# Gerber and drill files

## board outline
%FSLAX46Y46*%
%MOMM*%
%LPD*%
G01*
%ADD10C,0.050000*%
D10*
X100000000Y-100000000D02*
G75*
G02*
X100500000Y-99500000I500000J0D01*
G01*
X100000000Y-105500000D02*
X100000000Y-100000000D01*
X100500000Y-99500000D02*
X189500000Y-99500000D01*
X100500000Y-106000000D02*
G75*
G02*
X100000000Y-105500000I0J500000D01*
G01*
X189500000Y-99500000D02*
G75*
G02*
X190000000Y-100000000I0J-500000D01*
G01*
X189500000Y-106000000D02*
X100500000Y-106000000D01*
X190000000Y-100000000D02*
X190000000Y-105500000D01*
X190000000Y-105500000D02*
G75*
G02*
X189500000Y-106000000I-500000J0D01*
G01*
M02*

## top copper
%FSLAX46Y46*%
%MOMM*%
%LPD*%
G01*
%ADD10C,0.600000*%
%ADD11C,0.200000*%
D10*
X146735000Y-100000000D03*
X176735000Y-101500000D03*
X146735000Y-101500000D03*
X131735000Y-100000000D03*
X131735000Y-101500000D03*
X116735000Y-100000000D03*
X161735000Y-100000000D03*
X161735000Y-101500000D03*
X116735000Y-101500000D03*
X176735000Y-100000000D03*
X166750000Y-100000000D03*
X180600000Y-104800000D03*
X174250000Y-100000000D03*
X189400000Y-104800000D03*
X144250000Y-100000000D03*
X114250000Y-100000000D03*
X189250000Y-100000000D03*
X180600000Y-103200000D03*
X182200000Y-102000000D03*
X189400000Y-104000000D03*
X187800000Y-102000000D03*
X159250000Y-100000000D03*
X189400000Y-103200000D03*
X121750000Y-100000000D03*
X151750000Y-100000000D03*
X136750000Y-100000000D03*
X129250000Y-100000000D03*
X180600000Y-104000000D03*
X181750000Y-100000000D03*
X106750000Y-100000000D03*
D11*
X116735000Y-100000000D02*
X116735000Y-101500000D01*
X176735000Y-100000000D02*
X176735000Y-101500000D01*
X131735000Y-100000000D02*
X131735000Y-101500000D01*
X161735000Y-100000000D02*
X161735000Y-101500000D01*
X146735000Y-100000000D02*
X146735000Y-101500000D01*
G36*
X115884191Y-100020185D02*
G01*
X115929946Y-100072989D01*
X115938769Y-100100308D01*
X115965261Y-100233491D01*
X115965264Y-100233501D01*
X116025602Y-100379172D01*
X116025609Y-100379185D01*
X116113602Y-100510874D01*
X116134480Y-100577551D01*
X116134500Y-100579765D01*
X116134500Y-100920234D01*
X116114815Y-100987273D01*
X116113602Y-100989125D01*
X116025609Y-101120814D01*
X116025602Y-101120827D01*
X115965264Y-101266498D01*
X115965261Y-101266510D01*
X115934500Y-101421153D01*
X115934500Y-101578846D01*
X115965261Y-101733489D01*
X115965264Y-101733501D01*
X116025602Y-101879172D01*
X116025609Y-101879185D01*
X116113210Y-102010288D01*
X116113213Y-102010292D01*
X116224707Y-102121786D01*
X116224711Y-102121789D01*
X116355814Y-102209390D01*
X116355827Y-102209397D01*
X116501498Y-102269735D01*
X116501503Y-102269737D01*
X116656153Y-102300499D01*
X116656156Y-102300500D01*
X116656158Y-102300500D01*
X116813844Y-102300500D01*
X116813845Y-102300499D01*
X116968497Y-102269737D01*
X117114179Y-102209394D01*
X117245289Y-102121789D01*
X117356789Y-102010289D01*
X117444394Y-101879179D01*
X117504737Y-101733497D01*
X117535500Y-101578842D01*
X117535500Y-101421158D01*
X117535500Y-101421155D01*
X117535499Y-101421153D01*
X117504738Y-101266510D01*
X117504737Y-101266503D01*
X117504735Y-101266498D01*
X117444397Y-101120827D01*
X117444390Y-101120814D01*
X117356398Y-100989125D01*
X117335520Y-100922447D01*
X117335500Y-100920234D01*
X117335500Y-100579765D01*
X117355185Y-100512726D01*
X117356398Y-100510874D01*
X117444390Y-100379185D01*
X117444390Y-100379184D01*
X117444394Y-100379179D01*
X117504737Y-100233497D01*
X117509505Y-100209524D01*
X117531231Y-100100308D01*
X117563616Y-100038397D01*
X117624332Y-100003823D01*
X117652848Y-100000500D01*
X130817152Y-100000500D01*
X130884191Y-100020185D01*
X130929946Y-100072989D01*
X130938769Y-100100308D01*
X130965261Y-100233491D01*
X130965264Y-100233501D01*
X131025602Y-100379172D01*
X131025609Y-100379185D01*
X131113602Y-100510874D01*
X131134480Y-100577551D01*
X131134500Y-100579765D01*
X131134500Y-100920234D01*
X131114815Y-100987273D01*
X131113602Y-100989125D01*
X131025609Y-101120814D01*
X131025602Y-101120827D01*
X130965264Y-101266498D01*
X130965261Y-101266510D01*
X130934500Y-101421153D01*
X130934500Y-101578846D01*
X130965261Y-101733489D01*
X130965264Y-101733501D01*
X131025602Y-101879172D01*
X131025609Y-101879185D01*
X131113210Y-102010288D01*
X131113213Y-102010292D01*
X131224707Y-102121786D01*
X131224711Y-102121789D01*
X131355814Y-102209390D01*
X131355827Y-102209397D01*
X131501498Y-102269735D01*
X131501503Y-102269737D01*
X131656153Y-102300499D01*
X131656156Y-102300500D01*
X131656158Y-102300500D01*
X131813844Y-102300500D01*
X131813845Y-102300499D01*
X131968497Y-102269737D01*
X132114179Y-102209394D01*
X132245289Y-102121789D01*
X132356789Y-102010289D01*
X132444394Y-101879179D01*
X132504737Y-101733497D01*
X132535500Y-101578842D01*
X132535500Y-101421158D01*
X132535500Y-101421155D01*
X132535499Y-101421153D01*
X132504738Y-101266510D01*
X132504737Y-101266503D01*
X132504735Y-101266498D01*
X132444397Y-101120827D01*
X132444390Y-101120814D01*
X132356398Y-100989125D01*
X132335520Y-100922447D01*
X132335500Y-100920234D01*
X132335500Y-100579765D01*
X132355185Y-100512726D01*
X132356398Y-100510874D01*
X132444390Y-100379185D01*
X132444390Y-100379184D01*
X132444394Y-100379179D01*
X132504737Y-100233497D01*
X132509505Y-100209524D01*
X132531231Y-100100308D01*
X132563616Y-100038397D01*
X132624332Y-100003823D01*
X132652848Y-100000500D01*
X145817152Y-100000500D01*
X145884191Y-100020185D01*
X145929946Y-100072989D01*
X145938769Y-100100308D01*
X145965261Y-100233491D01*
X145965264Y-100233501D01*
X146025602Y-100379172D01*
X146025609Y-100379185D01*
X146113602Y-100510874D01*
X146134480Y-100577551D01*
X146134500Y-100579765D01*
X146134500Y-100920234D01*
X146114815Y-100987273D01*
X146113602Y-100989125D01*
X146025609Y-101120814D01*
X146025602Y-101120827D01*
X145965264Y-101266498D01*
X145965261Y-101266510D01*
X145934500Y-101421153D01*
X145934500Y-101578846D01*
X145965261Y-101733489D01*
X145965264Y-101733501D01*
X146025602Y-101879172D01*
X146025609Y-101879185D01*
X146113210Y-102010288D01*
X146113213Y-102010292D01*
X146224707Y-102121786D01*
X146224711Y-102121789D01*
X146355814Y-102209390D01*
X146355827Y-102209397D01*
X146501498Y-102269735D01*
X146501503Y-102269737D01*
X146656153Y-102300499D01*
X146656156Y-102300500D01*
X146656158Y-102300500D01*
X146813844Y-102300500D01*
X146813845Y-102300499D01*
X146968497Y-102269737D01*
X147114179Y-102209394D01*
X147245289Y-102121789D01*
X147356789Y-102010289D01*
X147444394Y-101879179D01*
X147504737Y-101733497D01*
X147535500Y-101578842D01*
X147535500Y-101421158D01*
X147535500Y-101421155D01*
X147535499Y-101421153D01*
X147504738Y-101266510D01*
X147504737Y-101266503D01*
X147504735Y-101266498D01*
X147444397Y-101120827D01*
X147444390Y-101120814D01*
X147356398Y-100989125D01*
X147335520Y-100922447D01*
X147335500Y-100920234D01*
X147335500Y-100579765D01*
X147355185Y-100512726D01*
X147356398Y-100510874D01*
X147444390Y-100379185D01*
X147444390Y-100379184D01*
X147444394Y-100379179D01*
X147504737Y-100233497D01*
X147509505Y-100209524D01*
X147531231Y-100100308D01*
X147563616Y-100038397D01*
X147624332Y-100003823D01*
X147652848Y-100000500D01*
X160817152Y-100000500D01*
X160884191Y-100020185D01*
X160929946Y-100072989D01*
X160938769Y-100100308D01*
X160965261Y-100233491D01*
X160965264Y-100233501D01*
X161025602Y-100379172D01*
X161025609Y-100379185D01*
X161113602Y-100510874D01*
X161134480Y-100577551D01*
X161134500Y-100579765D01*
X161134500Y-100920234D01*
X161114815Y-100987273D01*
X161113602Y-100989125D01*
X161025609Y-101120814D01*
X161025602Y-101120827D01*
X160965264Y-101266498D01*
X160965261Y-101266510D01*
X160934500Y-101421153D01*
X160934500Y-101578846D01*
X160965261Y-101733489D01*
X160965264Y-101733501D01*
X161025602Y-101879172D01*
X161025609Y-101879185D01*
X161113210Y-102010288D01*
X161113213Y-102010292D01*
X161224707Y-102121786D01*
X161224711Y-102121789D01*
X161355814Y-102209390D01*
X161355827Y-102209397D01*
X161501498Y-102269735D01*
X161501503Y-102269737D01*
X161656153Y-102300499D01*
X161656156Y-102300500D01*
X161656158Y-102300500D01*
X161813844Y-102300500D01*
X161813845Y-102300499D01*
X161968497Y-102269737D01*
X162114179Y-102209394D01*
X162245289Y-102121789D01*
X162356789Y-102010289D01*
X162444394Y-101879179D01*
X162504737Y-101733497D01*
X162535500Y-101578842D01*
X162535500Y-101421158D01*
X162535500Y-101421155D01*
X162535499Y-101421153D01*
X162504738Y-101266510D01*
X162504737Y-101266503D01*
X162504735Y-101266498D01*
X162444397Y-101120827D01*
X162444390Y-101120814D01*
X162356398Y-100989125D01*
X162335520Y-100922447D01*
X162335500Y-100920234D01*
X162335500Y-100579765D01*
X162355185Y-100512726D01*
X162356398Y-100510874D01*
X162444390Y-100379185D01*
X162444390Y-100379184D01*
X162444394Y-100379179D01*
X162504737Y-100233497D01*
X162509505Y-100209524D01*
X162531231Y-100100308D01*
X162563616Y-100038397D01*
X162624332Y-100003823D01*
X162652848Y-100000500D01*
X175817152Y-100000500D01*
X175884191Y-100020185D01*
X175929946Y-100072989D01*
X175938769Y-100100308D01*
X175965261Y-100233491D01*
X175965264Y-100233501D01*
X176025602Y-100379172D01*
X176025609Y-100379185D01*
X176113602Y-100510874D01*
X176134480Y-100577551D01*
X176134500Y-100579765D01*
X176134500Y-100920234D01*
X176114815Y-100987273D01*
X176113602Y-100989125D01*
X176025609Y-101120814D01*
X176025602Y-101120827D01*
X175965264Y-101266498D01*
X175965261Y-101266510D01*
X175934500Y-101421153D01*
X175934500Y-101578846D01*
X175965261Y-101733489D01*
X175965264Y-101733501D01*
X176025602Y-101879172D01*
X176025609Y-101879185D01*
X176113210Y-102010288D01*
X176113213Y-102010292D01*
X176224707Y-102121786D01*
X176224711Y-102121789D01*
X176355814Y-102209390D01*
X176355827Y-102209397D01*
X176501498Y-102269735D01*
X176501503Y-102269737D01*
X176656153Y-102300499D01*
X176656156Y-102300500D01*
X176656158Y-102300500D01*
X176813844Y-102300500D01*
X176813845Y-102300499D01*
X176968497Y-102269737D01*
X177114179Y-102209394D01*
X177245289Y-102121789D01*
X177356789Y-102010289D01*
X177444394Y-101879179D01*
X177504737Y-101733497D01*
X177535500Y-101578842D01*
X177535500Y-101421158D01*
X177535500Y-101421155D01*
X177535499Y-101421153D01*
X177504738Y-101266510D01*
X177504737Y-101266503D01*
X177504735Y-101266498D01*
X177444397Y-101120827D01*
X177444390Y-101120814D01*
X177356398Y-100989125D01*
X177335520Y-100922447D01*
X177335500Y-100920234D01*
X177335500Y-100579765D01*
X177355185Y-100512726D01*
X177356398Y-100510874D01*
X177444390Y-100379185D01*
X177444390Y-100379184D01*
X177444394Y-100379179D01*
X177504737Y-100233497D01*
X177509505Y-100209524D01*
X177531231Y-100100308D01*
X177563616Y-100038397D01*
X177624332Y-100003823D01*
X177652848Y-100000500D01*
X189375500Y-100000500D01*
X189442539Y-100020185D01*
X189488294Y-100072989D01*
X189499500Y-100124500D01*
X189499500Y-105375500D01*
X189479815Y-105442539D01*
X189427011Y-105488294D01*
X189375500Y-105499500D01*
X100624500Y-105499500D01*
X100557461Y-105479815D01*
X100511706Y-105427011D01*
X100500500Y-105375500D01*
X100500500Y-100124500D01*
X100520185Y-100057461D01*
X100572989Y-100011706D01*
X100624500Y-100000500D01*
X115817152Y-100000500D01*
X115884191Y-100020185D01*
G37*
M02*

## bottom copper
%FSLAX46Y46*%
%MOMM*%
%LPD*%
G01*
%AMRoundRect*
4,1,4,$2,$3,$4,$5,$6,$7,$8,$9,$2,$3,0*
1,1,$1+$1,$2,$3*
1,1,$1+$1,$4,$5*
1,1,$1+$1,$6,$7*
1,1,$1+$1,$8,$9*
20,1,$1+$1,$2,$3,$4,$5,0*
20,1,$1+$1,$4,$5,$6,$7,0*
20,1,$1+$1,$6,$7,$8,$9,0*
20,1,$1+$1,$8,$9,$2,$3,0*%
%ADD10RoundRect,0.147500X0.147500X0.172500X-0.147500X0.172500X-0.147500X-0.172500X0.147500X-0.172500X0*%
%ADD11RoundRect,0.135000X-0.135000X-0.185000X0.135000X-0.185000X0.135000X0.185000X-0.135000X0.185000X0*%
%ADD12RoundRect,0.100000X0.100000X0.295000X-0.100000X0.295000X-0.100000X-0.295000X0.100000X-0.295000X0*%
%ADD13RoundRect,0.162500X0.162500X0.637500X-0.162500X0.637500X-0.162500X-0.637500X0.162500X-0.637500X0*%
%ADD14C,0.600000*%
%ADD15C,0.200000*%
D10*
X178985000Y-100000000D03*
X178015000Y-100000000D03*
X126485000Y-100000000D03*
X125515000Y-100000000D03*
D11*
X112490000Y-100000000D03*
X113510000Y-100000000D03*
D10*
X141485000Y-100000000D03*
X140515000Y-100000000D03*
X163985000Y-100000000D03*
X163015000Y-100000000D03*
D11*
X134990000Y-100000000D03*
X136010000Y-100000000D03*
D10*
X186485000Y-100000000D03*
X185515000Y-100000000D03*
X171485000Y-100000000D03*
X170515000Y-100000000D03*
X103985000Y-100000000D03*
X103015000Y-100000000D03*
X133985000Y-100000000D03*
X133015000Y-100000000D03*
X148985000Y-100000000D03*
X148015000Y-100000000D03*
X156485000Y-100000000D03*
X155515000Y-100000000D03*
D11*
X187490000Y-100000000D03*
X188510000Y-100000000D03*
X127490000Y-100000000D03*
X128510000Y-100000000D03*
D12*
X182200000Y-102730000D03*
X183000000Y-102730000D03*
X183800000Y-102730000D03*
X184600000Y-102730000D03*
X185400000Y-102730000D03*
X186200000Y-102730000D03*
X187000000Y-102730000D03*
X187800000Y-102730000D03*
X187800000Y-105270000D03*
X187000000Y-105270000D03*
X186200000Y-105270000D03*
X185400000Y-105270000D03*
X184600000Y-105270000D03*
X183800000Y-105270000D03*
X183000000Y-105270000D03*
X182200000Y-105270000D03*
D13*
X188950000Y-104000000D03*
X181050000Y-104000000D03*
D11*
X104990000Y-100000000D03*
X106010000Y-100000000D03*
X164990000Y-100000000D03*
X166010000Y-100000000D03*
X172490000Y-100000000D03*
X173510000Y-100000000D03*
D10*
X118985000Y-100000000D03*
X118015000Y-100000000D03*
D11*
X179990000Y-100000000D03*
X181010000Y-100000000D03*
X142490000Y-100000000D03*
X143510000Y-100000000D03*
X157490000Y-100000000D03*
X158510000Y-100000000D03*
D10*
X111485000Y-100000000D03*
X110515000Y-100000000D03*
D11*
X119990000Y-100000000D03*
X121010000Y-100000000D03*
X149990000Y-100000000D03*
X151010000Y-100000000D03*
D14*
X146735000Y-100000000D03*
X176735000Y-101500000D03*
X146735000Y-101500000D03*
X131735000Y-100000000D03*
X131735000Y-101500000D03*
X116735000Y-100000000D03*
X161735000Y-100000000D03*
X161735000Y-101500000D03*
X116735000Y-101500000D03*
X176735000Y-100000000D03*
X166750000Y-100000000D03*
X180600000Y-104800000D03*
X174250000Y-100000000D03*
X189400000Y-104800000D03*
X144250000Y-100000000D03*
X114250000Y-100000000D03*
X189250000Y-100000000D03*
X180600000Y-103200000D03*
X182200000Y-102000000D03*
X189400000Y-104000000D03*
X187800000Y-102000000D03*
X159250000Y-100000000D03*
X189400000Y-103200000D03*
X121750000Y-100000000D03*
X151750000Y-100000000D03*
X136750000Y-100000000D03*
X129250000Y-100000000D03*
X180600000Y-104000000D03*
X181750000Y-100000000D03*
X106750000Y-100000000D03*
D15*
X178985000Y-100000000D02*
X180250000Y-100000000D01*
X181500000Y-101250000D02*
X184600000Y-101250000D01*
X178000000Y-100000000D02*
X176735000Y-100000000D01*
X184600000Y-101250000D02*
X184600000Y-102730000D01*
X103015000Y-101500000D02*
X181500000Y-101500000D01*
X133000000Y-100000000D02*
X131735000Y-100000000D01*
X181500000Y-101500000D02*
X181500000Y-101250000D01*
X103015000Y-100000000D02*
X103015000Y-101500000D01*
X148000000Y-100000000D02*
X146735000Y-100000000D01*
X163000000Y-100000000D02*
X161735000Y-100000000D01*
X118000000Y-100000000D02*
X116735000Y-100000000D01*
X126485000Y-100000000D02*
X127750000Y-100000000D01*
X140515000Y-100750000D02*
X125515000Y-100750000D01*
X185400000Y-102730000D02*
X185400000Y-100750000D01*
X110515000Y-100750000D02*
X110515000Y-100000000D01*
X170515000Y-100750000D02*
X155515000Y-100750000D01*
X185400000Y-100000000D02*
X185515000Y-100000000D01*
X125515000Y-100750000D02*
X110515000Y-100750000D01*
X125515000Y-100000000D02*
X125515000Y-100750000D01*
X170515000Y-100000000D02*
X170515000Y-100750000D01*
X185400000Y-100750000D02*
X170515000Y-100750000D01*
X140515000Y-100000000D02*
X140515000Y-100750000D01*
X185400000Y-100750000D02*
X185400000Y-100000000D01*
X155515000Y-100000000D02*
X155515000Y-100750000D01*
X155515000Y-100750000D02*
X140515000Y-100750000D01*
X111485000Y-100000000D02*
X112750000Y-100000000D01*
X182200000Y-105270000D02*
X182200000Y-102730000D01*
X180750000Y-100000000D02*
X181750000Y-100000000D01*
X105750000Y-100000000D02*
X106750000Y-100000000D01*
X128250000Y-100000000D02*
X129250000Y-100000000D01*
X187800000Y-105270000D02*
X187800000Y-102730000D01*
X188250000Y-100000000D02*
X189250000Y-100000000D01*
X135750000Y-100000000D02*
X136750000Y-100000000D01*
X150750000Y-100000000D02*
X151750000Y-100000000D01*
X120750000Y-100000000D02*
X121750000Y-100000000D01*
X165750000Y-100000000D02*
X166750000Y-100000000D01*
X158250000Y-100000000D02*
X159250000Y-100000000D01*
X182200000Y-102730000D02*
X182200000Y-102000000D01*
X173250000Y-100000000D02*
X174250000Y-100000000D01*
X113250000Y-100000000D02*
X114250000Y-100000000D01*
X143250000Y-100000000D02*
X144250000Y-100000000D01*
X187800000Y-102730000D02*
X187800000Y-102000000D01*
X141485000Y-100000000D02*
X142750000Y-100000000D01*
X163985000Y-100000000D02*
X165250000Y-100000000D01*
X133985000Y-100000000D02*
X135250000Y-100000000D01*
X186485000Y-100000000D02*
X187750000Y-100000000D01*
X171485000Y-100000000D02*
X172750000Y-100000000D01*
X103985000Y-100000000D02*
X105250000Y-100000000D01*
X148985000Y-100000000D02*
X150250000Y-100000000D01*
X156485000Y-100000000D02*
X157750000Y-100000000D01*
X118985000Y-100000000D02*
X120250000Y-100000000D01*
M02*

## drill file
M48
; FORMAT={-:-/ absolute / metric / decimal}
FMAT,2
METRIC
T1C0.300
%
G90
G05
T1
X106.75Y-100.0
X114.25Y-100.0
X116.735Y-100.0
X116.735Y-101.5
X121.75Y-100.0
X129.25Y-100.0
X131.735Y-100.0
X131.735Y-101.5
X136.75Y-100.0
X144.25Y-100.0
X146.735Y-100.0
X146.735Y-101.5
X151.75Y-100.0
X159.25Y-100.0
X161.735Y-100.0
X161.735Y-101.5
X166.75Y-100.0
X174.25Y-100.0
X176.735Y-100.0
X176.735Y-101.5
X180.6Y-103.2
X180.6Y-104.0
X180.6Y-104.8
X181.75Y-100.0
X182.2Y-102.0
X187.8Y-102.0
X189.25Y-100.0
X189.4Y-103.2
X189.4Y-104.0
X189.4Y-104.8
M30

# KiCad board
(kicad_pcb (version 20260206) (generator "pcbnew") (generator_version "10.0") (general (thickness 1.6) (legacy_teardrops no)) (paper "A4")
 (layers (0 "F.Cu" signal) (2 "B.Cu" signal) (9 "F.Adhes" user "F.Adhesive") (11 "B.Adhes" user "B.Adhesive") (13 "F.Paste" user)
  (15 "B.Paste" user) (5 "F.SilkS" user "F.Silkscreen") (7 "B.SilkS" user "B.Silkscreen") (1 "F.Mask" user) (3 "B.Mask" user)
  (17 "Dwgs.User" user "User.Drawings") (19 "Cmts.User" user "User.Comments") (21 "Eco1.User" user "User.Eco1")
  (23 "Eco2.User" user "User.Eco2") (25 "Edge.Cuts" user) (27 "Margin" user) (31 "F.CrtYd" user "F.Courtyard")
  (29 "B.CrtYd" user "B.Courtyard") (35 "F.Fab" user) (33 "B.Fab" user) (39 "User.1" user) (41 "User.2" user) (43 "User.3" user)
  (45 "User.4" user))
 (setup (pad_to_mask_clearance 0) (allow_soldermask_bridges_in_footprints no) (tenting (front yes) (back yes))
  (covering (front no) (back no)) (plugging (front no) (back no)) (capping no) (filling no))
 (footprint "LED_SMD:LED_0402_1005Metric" (layer "B.Cu") (at 178.5 100 180)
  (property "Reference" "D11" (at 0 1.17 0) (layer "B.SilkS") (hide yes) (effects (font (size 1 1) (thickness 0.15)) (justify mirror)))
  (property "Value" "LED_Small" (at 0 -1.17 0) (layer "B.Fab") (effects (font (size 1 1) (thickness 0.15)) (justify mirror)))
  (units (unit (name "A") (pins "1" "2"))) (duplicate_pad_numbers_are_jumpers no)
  (pad "1" smd roundrect (at -0.485 0 180) (size 0.59 0.64) (layers "B.Cu" "B.Mask" "B.Paste") (roundrect_rratio 0.25) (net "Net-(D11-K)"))
  (pad "2" smd roundrect (at 0.485 0 180) (size 0.59 0.64) (layers "B.Cu" "B.Mask" "B.Paste") (roundrect_rratio 0.25) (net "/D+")))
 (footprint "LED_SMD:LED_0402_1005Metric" (layer "B.Cu") (at 126 100 180)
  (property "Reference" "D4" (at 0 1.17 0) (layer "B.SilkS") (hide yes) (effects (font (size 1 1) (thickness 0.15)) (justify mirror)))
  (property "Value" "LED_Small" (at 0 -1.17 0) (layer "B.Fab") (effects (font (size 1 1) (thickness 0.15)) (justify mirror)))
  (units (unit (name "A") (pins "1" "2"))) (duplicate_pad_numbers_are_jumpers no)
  (pad "1" smd roundrect (at -0.485 0 180) (size 0.59 0.64) (layers "B.Cu" "B.Mask" "B.Paste") (roundrect_rratio 0.25) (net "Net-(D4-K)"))
  (pad "2" smd roundrect (at 0.485 0 180) (size 0.59 0.64) (layers "B.Cu" "B.Mask" "B.Paste") (roundrect_rratio 0.25) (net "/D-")))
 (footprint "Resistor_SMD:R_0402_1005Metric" (layer "B.Cu") (at 113 100)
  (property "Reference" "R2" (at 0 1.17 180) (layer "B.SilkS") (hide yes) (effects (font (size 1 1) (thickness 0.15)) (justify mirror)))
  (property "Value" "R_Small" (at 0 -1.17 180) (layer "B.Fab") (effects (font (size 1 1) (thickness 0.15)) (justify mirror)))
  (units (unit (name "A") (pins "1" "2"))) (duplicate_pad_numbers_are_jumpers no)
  (pad "1" smd roundrect (at -0.51 0) (size 0.54 0.64) (layers "B.Cu" "B.Mask" "B.Paste") (roundrect_rratio 0.25) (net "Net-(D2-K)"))
  (pad "2" smd roundrect (at 0.51 0) (size 0.54 0.64) (layers "B.Cu" "B.Mask" "B.Paste") (roundrect_rratio 0.25) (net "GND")))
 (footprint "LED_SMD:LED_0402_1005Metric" (layer "B.Cu") (at 141 100 180)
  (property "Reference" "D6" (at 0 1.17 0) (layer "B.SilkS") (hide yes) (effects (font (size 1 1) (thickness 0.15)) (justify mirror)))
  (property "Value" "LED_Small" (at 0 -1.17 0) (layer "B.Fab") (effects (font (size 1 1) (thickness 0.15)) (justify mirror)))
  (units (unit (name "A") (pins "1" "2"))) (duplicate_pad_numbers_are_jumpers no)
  (pad "1" smd roundrect (at -0.485 0 180) (size 0.59 0.64) (layers "B.Cu" "B.Mask" "B.Paste") (roundrect_rratio 0.25) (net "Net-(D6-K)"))
  (pad "2" smd roundrect (at 0.485 0 180) (size 0.59 0.64) (layers "B.Cu" "B.Mask" "B.Paste") (roundrect_rratio 0.25) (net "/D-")))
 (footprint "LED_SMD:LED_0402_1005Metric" (layer "B.Cu") (at 163.5 100 180)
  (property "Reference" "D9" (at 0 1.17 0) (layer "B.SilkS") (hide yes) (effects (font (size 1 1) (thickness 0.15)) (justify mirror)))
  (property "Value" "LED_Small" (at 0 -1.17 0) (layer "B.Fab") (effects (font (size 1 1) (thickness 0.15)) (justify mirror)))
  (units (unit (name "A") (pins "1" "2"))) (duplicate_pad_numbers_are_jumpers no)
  (pad "1" smd roundrect (at -0.485 0 180) (size 0.59 0.64) (layers "B.Cu" "B.Mask" "B.Paste") (roundrect_rratio 0.25) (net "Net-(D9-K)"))
  (pad "2" smd roundrect (at 0.485 0 180) (size 0.59 0.64) (layers "B.Cu" "B.Mask" "B.Paste") (roundrect_rratio 0.25) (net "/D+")))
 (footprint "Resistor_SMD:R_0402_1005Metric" (layer "B.Cu") (at 135.5 100)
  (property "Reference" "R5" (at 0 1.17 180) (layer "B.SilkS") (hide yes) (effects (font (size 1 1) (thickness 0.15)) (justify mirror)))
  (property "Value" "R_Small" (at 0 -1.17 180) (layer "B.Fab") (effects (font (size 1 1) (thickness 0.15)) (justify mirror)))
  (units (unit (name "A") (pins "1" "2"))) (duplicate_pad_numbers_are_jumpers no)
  (pad "1" smd roundrect (at -0.51 0) (size 0.54 0.64) (layers "B.Cu" "B.Mask" "B.Paste") (roundrect_rratio 0.25) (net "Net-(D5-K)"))
  (pad "2" smd roundrect (at 0.51 0) (size 0.54 0.64) (layers "B.Cu" "B.Mask" "B.Paste") (roundrect_rratio 0.25) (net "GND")))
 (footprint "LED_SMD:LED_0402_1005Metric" (layer "B.Cu") (at 186 100 180)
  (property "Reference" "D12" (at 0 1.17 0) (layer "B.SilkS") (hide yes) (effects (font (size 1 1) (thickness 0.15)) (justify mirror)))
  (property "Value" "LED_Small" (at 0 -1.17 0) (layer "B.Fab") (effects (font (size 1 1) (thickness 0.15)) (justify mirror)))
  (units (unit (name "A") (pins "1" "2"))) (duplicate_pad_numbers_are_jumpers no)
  (pad "1" smd roundrect (at -0.485 0 180) (size 0.59 0.64) (layers "B.Cu" "B.Mask" "B.Paste") (roundrect_rratio 0.25) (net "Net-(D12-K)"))
  (pad "2" smd roundrect (at 0.485 0 180) (size 0.59 0.64) (layers "B.Cu" "B.Mask" "B.Paste") (roundrect_rratio 0.25) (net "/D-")))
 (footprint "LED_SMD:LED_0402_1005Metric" (layer "B.Cu") (at 171 100 180)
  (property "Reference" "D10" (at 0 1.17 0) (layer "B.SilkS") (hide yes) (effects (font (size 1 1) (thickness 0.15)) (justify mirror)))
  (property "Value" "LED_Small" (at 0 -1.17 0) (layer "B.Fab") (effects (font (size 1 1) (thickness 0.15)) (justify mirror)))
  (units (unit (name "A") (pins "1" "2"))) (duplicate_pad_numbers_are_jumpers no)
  (pad "1" smd roundrect (at -0.485 0 180) (size 0.59 0.64) (layers "B.Cu" "B.Mask" "B.Paste") (roundrect_rratio 0.25) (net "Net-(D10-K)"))
  (pad "2" smd roundrect (at 0.485 0 180) (size 0.59 0.64) (layers "B.Cu" "B.Mask" "B.Paste") (roundrect_rratio 0.25) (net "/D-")))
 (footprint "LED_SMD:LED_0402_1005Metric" (layer "B.Cu") (at 103.5 100 180)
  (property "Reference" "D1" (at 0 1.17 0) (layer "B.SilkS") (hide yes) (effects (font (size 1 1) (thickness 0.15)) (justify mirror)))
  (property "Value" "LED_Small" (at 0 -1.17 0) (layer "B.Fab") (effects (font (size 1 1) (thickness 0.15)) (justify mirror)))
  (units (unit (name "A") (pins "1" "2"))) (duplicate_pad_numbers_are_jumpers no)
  (pad "1" smd roundrect (at -0.485 0 180) (size 0.59 0.64) (layers "B.Cu" "B.Mask" "B.Paste") (roundrect_rratio 0.25) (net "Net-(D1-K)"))
  (pad "2" smd roundrect (at 0.485 0 180) (size 0.59 0.64) (layers "B.Cu" "B.Mask" "B.Paste") (roundrect_rratio 0.25) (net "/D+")))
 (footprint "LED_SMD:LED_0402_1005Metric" (layer "B.Cu") (at 133.5 100 180)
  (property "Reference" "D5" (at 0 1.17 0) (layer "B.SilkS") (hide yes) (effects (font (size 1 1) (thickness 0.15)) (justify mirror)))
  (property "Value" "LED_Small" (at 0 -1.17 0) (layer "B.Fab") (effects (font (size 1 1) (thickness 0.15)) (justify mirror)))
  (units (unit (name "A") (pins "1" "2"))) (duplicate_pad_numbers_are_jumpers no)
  (pad "1" smd roundrect (at -0.485 0 180) (size 0.59 0.64) (layers "B.Cu" "B.Mask" "B.Paste") (roundrect_rratio 0.25) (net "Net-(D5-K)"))
  (pad "2" smd roundrect (at 0.485 0 180) (size 0.59 0.64) (layers "B.Cu" "B.Mask" "B.Paste") (roundrect_rratio 0.25) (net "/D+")))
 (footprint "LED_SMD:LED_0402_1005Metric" (layer "B.Cu") (at 148.5 100 180)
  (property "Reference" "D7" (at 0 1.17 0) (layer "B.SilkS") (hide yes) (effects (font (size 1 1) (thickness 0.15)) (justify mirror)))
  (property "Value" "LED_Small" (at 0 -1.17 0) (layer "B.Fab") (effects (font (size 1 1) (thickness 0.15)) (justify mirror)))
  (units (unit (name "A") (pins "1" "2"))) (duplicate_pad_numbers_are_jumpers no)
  (pad "1" smd roundrect (at -0.485 0 180) (size 0.59 0.64) (layers "B.Cu" "B.Mask" "B.Paste") (roundrect_rratio 0.25) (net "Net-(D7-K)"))
  (pad "2" smd roundrect (at 0.485 0 180) (size 0.59 0.64) (layers "B.Cu" "B.Mask" "B.Paste") (roundrect_rratio 0.25) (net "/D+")))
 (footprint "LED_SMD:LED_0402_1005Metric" (layer "B.Cu") (at 156 100 180)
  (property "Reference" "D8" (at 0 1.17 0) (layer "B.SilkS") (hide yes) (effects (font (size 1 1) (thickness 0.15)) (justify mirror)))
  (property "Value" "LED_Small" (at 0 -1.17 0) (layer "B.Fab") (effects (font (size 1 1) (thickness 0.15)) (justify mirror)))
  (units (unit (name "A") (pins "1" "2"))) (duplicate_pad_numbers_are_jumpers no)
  (pad "1" smd roundrect (at -0.485 0 180) (size 0.59 0.64) (layers "B.Cu" "B.Mask" "B.Paste") (roundrect_rratio 0.25) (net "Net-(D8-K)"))
  (pad "2" smd roundrect (at 0.485 0 180) (size 0.59 0.64) (layers "B.Cu" "B.Mask" "B.Paste") (roundrect_rratio 0.25) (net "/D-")))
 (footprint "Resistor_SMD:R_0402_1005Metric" (layer "B.Cu") (at 188 100)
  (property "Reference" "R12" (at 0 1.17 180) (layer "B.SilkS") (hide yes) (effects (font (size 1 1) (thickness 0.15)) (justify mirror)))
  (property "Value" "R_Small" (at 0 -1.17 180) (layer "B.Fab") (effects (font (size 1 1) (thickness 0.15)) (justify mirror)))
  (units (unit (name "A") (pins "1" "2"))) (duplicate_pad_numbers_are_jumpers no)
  (pad "1" smd roundrect (at -0.51 0) (size 0.54 0.64) (layers "B.Cu" "B.Mask" "B.Paste") (roundrect_rratio 0.25) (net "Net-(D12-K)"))
  (pad "2" smd roundrect (at 0.51 0) (size 0.54 0.64) (layers "B.Cu" "B.Mask" "B.Paste") (roundrect_rratio 0.25) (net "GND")))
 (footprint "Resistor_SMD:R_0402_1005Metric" (layer "B.Cu") (at 128 100)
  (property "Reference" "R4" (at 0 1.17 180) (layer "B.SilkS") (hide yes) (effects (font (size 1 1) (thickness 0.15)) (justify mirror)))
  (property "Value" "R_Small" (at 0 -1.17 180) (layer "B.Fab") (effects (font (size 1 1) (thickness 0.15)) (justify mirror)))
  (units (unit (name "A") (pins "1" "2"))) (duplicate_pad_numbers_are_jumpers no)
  (pad "1" smd roundrect (at -0.51 0) (size 0.54 0.64) (layers "B.Cu" "B.Mask" "B.Paste") (roundrect_rratio 0.25) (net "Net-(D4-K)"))
  (pad "2" smd roundrect (at 0.51 0) (size 0.54 0.64) (layers "B.Cu" "B.Mask" "B.Paste") (roundrect_rratio 0.25) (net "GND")))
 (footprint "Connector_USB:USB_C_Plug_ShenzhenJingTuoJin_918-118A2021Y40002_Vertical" (layer "B.Cu") (at 185 104 -90)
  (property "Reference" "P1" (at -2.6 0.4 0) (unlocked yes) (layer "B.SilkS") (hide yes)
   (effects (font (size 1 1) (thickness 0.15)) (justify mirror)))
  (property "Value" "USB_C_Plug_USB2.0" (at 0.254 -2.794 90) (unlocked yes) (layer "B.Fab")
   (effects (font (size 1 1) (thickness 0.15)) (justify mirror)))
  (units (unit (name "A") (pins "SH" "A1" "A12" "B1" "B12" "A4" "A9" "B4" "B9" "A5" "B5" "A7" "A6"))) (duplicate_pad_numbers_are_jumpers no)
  (pad "A1" smd roundrect (at -1.27 2.8 180) (size 0.4 0.79) (layers "B.Cu" "B.Mask" "B.Paste") (roundrect_rratio 0.25) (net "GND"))
  (pad "A4" smd roundrect (at -1.27 2 180) (size 0.4 0.79) (layers "B.Cu" "B.Mask" "B.Paste") (roundrect_rratio 0.25)
   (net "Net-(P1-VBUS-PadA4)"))
  (pad "A5" smd roundrect (at -1.27 1.2 180) (size 0.4 0.79) (layers "B.Cu" "B.Mask" "B.Paste") (roundrect_rratio 0.25)
   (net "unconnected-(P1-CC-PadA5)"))
  (pad "A6" smd roundrect (at -1.27 0.4 180) (size 0.4 0.79) (layers "B.Cu" "B.Mask" "B.Paste") (roundrect_rratio 0.25) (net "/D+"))
  (pad "A7" smd roundrect (at -1.27 -0.4 180) (size 0.4 0.79) (layers "B.Cu" "B.Mask" "B.Paste") (roundrect_rratio 0.25) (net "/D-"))
  (pad "A8" smd roundrect (at -1.27 -1.2 180) (size 0.4 0.79) (layers "B.Cu" "B.Mask" "B.Paste") (roundrect_rratio 0.25))
  (pad "A9" smd roundrect (at -1.27 -2 180) (size 0.4 0.79) (layers "B.Cu" "B.Mask" "B.Paste") (roundrect_rratio 0.25)
   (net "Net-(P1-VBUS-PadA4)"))
  (pad "A12" smd roundrect (at -1.27 -2.8 180) (size 0.4 0.79) (layers "B.Cu" "B.Mask" "B.Paste") (roundrect_rratio 0.25) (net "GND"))
  (pad "B1" smd roundrect (at 1.27 -2.8 180) (size 0.4 0.79) (layers "B.Cu" "B.Mask" "B.Paste") (roundrect_rratio 0.25) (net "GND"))
  (pad "B4" smd roundrect (at 1.27 -2 180) (size 0.4 0.79) (layers "B.Cu" "B.Mask" "B.Paste") (roundrect_rratio 0.25)
   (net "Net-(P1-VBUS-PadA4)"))
  (pad "B5" smd roundrect (at 1.27 -1.2 180) (size 0.4 0.79) (layers "B.Cu" "B.Mask" "B.Paste") (roundrect_rratio 0.25)
   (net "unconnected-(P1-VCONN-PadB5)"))
  (pad "B6" smd roundrect (at 1.27 -0.4 180) (size 0.4 0.79) (layers "B.Cu" "B.Mask" "B.Paste") (roundrect_rratio 0.25))
  (pad "B7" smd roundrect (at 1.27 0.4 180) (size 0.4 0.79) (layers "B.Cu" "B.Mask" "B.Paste") (roundrect_rratio 0.25))
  (pad "B8" smd roundrect (at 1.27 1.2 180) (size 0.4 0.79) (layers "B.Cu" "B.Mask" "B.Paste") (roundrect_rratio 0.25))
  (pad "B9" smd roundrect (at 1.27 2 180) (size 0.4 0.79) (layers "B.Cu" "B.Mask" "B.Paste") (roundrect_rratio 0.25)
   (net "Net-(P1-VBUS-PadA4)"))
  (pad "B12" smd roundrect (at 1.27 2.8 180) (size 0.4 0.79) (layers "B.Cu" "B.Mask" "B.Paste") (roundrect_rratio 0.25) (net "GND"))
  (pad "SH" smd roundrect (at 0 -3.95 180) (size 0.65 1.6) (layers "B.Cu" "B.Mask" "B.Paste") (roundrect_rratio 0.25) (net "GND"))
  (pad "SH" smd roundrect (at 0 3.95 180) (size 0.65 1.6) (layers "B.Cu" "B.Mask" "B.Paste") (roundrect_rratio 0.25) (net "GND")))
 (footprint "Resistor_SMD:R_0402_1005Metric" (layer "B.Cu") (at 105.5 100)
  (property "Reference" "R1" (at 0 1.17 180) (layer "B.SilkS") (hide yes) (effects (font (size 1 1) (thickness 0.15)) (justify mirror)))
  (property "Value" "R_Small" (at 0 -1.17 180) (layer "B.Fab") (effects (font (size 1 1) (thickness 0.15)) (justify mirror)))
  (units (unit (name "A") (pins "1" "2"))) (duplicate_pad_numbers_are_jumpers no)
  (pad "1" smd roundrect (at -0.51 0) (size 0.54 0.64) (layers "B.Cu" "B.Mask" "B.Paste") (roundrect_rratio 0.25) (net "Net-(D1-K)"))
  (pad "2" smd roundrect (at 0.51 0) (size 0.54 0.64) (layers "B.Cu" "B.Mask" "B.Paste") (roundrect_rratio 0.25) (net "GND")))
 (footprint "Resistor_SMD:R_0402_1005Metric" (layer "B.Cu") (at 165.5 100)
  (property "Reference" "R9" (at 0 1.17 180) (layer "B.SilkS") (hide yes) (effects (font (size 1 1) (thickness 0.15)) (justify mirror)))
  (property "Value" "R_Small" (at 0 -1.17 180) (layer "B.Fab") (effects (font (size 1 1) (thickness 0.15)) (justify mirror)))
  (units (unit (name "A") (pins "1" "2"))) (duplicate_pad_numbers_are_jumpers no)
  (pad "1" smd roundrect (at -0.51 0) (size 0.54 0.64) (layers "B.Cu" "B.Mask" "B.Paste") (roundrect_rratio 0.25) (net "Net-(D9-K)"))
  (pad "2" smd roundrect (at 0.51 0) (size 0.54 0.64) (layers "B.Cu" "B.Mask" "B.Paste") (roundrect_rratio 0.25) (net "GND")))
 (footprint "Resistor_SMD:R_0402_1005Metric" (layer "B.Cu") (at 173 100)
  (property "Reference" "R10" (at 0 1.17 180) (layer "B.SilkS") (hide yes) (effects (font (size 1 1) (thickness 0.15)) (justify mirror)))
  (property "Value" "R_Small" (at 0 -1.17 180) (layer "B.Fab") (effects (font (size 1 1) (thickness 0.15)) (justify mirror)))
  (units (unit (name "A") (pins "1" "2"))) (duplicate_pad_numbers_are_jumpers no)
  (pad "1" smd roundrect (at -0.51 0) (size 0.54 0.64) (layers "B.Cu" "B.Mask" "B.Paste") (roundrect_rratio 0.25) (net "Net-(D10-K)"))
  (pad "2" smd roundrect (at 0.51 0) (size 0.54 0.64) (layers "B.Cu" "B.Mask" "B.Paste") (roundrect_rratio 0.25) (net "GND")))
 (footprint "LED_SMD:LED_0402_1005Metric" (layer "B.Cu") (at 118.5 100 180)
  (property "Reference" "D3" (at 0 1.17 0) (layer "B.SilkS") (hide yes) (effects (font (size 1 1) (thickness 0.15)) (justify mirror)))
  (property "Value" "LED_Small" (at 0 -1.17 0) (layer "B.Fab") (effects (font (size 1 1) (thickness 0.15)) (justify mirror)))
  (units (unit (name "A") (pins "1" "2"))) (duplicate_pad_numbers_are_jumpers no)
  (pad "1" smd roundrect (at -0.485 0 180) (size 0.59 0.64) (layers "B.Cu" "B.Mask" "B.Paste") (roundrect_rratio 0.25) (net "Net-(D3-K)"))
  (pad "2" smd roundrect (at 0.485 0 180) (size 0.59 0.64) (layers "B.Cu" "B.Mask" "B.Paste") (roundrect_rratio 0.25) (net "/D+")))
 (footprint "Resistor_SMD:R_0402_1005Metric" (layer "B.Cu") (at 180.5 100)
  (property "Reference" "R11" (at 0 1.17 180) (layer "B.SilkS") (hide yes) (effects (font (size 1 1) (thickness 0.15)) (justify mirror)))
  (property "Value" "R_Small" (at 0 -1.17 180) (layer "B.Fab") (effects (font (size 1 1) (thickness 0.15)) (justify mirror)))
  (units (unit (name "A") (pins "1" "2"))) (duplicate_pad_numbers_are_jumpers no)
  (pad "1" smd roundrect (at -0.51 0) (size 0.54 0.64) (layers "B.Cu" "B.Mask" "B.Paste") (roundrect_rratio 0.25) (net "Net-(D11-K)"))
  (pad "2" smd roundrect (at 0.51 0) (size 0.54 0.64) (layers "B.Cu" "B.Mask" "B.Paste") (roundrect_rratio 0.25) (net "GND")))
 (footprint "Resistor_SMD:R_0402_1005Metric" (layer "B.Cu") (at 143 100)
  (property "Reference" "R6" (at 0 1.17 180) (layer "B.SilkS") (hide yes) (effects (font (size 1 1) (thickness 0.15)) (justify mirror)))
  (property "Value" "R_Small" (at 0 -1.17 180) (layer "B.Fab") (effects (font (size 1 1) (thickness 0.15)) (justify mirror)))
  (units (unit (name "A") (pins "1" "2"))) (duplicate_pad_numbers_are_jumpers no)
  (pad "1" smd roundrect (at -0.51 0) (size 0.54 0.64) (layers "B.Cu" "B.Mask" "B.Paste") (roundrect_rratio 0.25) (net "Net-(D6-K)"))
  (pad "2" smd roundrect (at 0.51 0) (size 0.54 0.64) (layers "B.Cu" "B.Mask" "B.Paste") (roundrect_rratio 0.25) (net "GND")))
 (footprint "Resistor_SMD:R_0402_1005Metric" (layer "B.Cu") (at 158 100)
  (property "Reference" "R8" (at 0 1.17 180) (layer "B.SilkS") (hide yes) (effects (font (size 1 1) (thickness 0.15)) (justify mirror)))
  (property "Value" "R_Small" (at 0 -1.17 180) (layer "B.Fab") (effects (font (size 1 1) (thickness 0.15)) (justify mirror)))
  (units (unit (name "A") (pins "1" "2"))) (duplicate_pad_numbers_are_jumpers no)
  (pad "1" smd roundrect (at -0.51 0) (size 0.54 0.64) (layers "B.Cu" "B.Mask" "B.Paste") (roundrect_rratio 0.25) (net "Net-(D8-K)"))
  (pad "2" smd roundrect (at 0.51 0) (size 0.54 0.64) (layers "B.Cu" "B.Mask" "B.Paste") (roundrect_rratio 0.25) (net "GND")))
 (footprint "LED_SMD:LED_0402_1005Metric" (layer "B.Cu") (at 111 100 180)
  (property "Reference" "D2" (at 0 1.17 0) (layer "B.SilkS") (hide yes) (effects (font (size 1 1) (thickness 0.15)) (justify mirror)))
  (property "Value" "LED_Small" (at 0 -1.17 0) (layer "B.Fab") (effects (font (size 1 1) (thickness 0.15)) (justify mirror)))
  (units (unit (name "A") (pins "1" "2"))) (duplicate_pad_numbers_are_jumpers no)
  (pad "1" smd roundrect (at -0.485 0 180) (size 0.59 0.64) (layers "B.Cu" "B.Mask" "B.Paste") (roundrect_rratio 0.25) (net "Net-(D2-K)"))
  (pad "2" smd roundrect (at 0.485 0 180) (size 0.59 0.64) (layers "B.Cu" "B.Mask" "B.Paste") (roundrect_rratio 0.25) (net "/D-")))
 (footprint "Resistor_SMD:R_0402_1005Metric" (layer "B.Cu") (at 120.5 100)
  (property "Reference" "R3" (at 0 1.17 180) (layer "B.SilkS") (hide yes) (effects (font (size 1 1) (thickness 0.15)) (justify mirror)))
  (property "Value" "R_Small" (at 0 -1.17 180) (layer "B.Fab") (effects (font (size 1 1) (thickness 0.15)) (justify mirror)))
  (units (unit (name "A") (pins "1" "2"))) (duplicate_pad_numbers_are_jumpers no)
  (pad "1" smd roundrect (at -0.51 0) (size 0.54 0.64) (layers "B.Cu" "B.Mask" "B.Paste") (roundrect_rratio 0.25) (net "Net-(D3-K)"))
  (pad "2" smd roundrect (at 0.51 0) (size 0.54 0.64) (layers "B.Cu" "B.Mask" "B.Paste") (roundrect_rratio 0.25) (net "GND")))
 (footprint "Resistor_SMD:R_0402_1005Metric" (layer "B.Cu") (at 150.5 100)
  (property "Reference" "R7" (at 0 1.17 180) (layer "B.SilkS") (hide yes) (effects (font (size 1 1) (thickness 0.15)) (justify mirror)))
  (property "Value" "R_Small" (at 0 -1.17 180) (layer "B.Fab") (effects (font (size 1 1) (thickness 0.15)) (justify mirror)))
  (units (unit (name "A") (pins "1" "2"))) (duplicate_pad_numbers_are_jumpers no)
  (pad "1" smd roundrect (at -0.51 0) (size 0.54 0.64) (layers "B.Cu" "B.Mask" "B.Paste") (roundrect_rratio 0.25) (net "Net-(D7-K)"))
  (pad "2" smd roundrect (at 0.51 0) (size 0.54 0.64) (layers "B.Cu" "B.Mask" "B.Paste") (roundrect_rratio 0.25) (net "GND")))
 (gr_arc (start 100 100) (mid 100.146447 99.646447) (end 100.5 99.5) (stroke (width 0.05) (type default)) (layer "Edge.Cuts"))
 (gr_line (start 100 105.5) (end 100 100) (stroke (width 0.05) (type default)) (layer "Edge.Cuts"))
 (gr_line (start 100.5 99.5) (end 189.5 99.5) (stroke (width 0.05) (type default)) (layer "Edge.Cuts"))
 (gr_arc (start 100.5 106) (mid 100.146447 105.853553) (end 100 105.5) (stroke (width 0.05) (type default)) (layer "Edge.Cuts"))
 (gr_arc (start 189.5 99.5) (mid 189.853553 99.646447) (end 190 100) (stroke (width 0.05) (type default)) (layer "Edge.Cuts"))
 (gr_line (start 189.5 106) (end 100.5 106) (stroke (width 0.05) (type default)) (layer "Edge.Cuts"))
 (gr_line (start 190 100) (end 190 105.5) (stroke (width 0.05) (type default)) (layer "Edge.Cuts"))
 (gr_arc (start 190 105.5) (mid 189.853553 105.853553) (end 189.5 106) (stroke (width 0.05) (type default)) (layer "Edge.Cuts"))
 (segment (start 178.985 100) (end 180.25 100) (width 0.2) (layer "B.Cu") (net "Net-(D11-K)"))
 (segment (start 116.735 100) (end 116.735 101.5) (width 0.2) (layer "F.Cu") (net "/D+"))
 (segment (start 176.735 100) (end 176.735 101.5) (width 0.2) (layer "F.Cu") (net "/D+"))
 (segment (start 131.735 100) (end 131.735 101.5) (width 0.2) (layer "F.Cu") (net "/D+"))
 (segment (start 161.735 100) (end 161.735 101.5) (width 0.2) (layer "F.Cu") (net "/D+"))
 (segment (start 146.735 100) (end 146.735 101.5) (width 0.2) (layer "F.Cu") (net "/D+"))
 (via (at 146.735 100) (size 0.6) (drill 0.3) (layers "F.Cu" "B.Cu") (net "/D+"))
 (via (at 176.735 101.5) (size 0.6) (drill 0.3) (layers "F.Cu" "B.Cu") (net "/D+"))
 (via (at 146.735 101.5) (size 0.6) (drill 0.3) (layers "F.Cu" "B.Cu") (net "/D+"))
 (via (at 131.735 100) (size 0.6) (drill 0.3) (layers "F.Cu" "B.Cu") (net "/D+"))
 (via (at 131.735 101.5) (size 0.6) (drill 0.3) (layers "F.Cu" "B.Cu") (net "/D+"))
 (via (at 116.735 100) (size 0.6) (drill 0.3) (layers "F.Cu" "B.Cu") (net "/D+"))
 (via (at 161.735 100) (size 0.6) (drill 0.3) (layers "F.Cu" "B.Cu") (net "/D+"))
 (via (at 161.735 101.5) (size 0.6) (drill 0.3) (layers "F.Cu" "B.Cu") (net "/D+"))
 (via (at 116.735 101.5) (size 0.6) (drill 0.3) (layers "F.Cu" "B.Cu") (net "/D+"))
 (via (at 176.735 100) (size 0.6) (drill 0.3) (layers "F.Cu" "B.Cu") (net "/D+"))
 (segment (start 181.5 101.25) (end 184.6 101.25) (width 0.2) (layer "B.Cu") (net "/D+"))
 (segment (start 178 100) (end 176.735 100) (width 0.2) (layer "B.Cu") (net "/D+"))
 (segment (start 184.6 101.25) (end 184.6 102.73) (width 0.2) (layer "B.Cu") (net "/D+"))
 (segment (start 103.015 101.5) (end 181.5 101.5) (width 0.2) (layer "B.Cu") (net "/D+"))
 (segment (start 133 100) (end 131.735 100) (width 0.2) (layer "B.Cu") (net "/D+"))
 (segment (start 181.5 101.5) (end 181.5 101.25) (width 0.2) (layer "B.Cu") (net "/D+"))
 (segment (start 103.015 100) (end 103.015 101.5) (width 0.2) (layer "B.Cu") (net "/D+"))
 (segment (start 148 100) (end 146.735 100) (width 0.2) (layer "B.Cu") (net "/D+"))
 (segment (start 163 100) (end 161.735 100) (width 0.2) (layer "B.Cu") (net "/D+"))
 (segment (start 118 100) (end 116.735 100) (width 0.2) (layer "B.Cu") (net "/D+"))
 (segment (start 126.485 100) (end 127.75 100) (width 0.2) (layer "B.Cu") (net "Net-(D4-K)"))
 (segment (start 140.515 100.75) (end 125.515 100.75) (width 0.2) (layer "B.Cu") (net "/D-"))
 (segment (start 185.4 102.73) (end 185.4 100.75) (width 0.2) (layer "B.Cu") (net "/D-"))
 (segment (start 110.515 100.75) (end 110.515 100) (width 0.2) (layer "B.Cu") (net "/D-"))
 (segment (start 170.515 100.75) (end 155.515 100.75) (width 0.2) (layer "B.Cu") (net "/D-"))
 (segment (start 185.4 100) (end 185.515 100) (width 0.2) (layer "B.Cu") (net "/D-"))
 (segment (start 125.515 100.75) (end 110.515 100.75) (width 0.2) (layer "B.Cu") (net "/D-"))
 (segment (start 125.515 100) (end 125.515 100.75) (width 0.2) (layer "B.Cu") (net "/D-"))
 (segment (start 170.515 100) (end 170.515 100.75) (width 0.2) (layer "B.Cu") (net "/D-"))
 (segment (start 185.4 100.75) (end 170.515 100.75) (width 0.2) (layer "B.Cu") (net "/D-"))
 (segment (start 140.515 100) (end 140.515 100.75) (width 0.2) (layer "B.Cu") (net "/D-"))
 (segment (start 185.4 100.75) (end 185.4 100) (width 0.2) (layer "B.Cu") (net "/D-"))
 (segment (start 155.515 100) (end 155.515 100.75) (width 0.2) (layer "B.Cu") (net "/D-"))
 (segment (start 155.515 100.75) (end 140.515 100.75) (width 0.2) (layer "B.Cu") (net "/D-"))
 (segment (start 111.485 100) (end 112.75 100) (width 0.2) (layer "B.Cu") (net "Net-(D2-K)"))
 (via (at 166.75 100) (size 0.6) (drill 0.3) (layers "F.Cu" "B.Cu") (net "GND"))
 (via (at 180.6 104.8) (size 0.6) (drill 0.3) (layers "F.Cu" "B.Cu") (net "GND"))
 (via (at 174.25 100) (size 0.6) (drill 0.3) (layers "F.Cu" "B.Cu") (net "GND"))
 (via (at 189.4 104.8) (size 0.6) (drill 0.3) (layers "F.Cu" "B.Cu") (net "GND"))
 (via (at 144.25 100) (size 0.6) (drill 0.3) (layers "F.Cu" "B.Cu") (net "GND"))
 (via (at 114.25 100) (size 0.6) (drill 0.3) (layers "F.Cu" "B.Cu") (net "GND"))
 (via (at 189.25 100) (size 0.6) (drill 0.3) (layers "F.Cu" "B.Cu") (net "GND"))
 (via (at 180.6 103.2) (size 0.6) (drill 0.3) (layers "F.Cu" "B.Cu") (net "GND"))
 (via (at 182.2 102) (size 0.6) (drill 0.3) (layers "F.Cu" "B.Cu") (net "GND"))
 (via (at 189.4 104) (size 0.6) (drill 0.3) (layers "F.Cu" "B.Cu") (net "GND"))
 (via (at 187.8 102) (size 0.6) (drill 0.3) (layers "F.Cu" "B.Cu") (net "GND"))
 (via (at 159.25 100) (size 0.6) (drill 0.3) (layers "F.Cu" "B.Cu") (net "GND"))
 (via (at 189.4 103.2) (size 0.6) (drill 0.3) (layers "F.Cu" "B.Cu") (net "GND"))
 (via (at 121.75 100) (size 0.6) (drill 0.3) (layers "F.Cu" "B.Cu") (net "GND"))
 (via (at 151.75 100) (size 0.6) (drill 0.3) (layers "F.Cu" "B.Cu") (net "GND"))
 (via (at 136.75 100) (size 0.6) (drill 0.3) (layers "F.Cu" "B.Cu") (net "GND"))
 (via (at 129.25 100) (size 0.6) (drill 0.3) (layers "F.Cu" "B.Cu") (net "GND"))
 (via (at 180.6 104) (size 0.6) (drill 0.3) (layers "F.Cu" "B.Cu") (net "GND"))
 (via (at 181.75 100) (size 0.6) (drill 0.3) (layers "F.Cu" "B.Cu") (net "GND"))
 (via (at 106.75 100) (size 0.6) (drill 0.3) (layers "F.Cu" "B.Cu") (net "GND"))
 (segment (start 182.2 105.27) (end 182.2 102.73) (width 0.2) (layer "B.Cu") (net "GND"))
 (segment (start 180.75 100) (end 181.75 100) (width 0.2) (layer "B.Cu") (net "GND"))
 (segment (start 105.75 100) (end 106.75 100) (width 0.2) (layer "B.Cu") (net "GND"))
 (segment (start 128.25 100) (end 129.25 100) (width 0.2) (layer "B.Cu") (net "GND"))
 (segment (start 187.8 105.27) (end 187.8 102.73) (width 0.2) (layer "B.Cu") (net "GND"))
 (segment (start 188.25 100) (end 189.25 100) (width 0.2) (layer "B.Cu") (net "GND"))
 (segment (start 135.75 100) (end 136.75 100) (width 0.2) (layer "B.Cu") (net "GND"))
 (segment (start 150.75 100) (end 151.75 100) (width 0.2) (layer "B.Cu") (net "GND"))
 (segment (start 120.75 100) (end 121.75 100) (width 0.2) (layer "B.Cu") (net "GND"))
 (segment (start 165.75 100) (end 166.75 100) (width 0.2) (layer "B.Cu") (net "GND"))
 (segment (start 158.25 100) (end 159.25 100) (width 0.2) (layer "B.Cu") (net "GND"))
 (segment (start 182.2 102.73) (end 182.2 102) (width 0.2) (layer "B.Cu") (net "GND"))
 (segment (start 173.25 100) (end 174.25 100) (width 0.2) (layer "B.Cu") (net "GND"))
 (segment (start 113.25 100) (end 114.25 100) (width 0.2) (layer "B.Cu") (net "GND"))
 (segment (start 143.25 100) (end 144.25 100) (width 0.2) (layer "B.Cu") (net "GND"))
 (segment (start 187.8 102.73) (end 187.8 102) (width 0.2) (layer "B.Cu") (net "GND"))
 (segment (start 141.485 100) (end 142.75 100) (width 0.2) (layer "B.Cu") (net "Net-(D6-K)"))
 (segment (start 163.985 100) (end 165.25 100) (width 0.2) (layer "B.Cu") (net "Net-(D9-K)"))
 (segment (start 133.985 100) (end 135.25 100) (width 0.2) (layer "B.Cu") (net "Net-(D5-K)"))
 (segment (start 186.485 100) (end 187.75 100) (width 0.2) (layer "B.Cu") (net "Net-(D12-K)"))
 (segment (start 171.485 100) (end 172.75 100) (width 0.2) (layer "B.Cu") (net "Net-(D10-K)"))
 (segment (start 103.985 100) (end 105.25 100) (width 0.2) (layer "B.Cu") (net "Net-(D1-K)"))
 (segment (start 148.985 100) (end 150.25 100) (width 0.2) (layer "B.Cu") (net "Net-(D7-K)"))
 (segment (start 156.485 100) (end 157.75 100) (width 0.2) (layer "B.Cu") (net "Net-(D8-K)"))
 (segment (start 118.985 100) (end 120.25 100) (width 0.2) (layer "B.Cu") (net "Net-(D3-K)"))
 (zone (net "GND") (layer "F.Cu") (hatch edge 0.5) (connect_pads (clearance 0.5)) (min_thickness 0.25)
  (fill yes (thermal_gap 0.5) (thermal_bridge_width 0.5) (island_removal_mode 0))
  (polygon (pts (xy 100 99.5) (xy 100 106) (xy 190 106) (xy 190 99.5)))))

